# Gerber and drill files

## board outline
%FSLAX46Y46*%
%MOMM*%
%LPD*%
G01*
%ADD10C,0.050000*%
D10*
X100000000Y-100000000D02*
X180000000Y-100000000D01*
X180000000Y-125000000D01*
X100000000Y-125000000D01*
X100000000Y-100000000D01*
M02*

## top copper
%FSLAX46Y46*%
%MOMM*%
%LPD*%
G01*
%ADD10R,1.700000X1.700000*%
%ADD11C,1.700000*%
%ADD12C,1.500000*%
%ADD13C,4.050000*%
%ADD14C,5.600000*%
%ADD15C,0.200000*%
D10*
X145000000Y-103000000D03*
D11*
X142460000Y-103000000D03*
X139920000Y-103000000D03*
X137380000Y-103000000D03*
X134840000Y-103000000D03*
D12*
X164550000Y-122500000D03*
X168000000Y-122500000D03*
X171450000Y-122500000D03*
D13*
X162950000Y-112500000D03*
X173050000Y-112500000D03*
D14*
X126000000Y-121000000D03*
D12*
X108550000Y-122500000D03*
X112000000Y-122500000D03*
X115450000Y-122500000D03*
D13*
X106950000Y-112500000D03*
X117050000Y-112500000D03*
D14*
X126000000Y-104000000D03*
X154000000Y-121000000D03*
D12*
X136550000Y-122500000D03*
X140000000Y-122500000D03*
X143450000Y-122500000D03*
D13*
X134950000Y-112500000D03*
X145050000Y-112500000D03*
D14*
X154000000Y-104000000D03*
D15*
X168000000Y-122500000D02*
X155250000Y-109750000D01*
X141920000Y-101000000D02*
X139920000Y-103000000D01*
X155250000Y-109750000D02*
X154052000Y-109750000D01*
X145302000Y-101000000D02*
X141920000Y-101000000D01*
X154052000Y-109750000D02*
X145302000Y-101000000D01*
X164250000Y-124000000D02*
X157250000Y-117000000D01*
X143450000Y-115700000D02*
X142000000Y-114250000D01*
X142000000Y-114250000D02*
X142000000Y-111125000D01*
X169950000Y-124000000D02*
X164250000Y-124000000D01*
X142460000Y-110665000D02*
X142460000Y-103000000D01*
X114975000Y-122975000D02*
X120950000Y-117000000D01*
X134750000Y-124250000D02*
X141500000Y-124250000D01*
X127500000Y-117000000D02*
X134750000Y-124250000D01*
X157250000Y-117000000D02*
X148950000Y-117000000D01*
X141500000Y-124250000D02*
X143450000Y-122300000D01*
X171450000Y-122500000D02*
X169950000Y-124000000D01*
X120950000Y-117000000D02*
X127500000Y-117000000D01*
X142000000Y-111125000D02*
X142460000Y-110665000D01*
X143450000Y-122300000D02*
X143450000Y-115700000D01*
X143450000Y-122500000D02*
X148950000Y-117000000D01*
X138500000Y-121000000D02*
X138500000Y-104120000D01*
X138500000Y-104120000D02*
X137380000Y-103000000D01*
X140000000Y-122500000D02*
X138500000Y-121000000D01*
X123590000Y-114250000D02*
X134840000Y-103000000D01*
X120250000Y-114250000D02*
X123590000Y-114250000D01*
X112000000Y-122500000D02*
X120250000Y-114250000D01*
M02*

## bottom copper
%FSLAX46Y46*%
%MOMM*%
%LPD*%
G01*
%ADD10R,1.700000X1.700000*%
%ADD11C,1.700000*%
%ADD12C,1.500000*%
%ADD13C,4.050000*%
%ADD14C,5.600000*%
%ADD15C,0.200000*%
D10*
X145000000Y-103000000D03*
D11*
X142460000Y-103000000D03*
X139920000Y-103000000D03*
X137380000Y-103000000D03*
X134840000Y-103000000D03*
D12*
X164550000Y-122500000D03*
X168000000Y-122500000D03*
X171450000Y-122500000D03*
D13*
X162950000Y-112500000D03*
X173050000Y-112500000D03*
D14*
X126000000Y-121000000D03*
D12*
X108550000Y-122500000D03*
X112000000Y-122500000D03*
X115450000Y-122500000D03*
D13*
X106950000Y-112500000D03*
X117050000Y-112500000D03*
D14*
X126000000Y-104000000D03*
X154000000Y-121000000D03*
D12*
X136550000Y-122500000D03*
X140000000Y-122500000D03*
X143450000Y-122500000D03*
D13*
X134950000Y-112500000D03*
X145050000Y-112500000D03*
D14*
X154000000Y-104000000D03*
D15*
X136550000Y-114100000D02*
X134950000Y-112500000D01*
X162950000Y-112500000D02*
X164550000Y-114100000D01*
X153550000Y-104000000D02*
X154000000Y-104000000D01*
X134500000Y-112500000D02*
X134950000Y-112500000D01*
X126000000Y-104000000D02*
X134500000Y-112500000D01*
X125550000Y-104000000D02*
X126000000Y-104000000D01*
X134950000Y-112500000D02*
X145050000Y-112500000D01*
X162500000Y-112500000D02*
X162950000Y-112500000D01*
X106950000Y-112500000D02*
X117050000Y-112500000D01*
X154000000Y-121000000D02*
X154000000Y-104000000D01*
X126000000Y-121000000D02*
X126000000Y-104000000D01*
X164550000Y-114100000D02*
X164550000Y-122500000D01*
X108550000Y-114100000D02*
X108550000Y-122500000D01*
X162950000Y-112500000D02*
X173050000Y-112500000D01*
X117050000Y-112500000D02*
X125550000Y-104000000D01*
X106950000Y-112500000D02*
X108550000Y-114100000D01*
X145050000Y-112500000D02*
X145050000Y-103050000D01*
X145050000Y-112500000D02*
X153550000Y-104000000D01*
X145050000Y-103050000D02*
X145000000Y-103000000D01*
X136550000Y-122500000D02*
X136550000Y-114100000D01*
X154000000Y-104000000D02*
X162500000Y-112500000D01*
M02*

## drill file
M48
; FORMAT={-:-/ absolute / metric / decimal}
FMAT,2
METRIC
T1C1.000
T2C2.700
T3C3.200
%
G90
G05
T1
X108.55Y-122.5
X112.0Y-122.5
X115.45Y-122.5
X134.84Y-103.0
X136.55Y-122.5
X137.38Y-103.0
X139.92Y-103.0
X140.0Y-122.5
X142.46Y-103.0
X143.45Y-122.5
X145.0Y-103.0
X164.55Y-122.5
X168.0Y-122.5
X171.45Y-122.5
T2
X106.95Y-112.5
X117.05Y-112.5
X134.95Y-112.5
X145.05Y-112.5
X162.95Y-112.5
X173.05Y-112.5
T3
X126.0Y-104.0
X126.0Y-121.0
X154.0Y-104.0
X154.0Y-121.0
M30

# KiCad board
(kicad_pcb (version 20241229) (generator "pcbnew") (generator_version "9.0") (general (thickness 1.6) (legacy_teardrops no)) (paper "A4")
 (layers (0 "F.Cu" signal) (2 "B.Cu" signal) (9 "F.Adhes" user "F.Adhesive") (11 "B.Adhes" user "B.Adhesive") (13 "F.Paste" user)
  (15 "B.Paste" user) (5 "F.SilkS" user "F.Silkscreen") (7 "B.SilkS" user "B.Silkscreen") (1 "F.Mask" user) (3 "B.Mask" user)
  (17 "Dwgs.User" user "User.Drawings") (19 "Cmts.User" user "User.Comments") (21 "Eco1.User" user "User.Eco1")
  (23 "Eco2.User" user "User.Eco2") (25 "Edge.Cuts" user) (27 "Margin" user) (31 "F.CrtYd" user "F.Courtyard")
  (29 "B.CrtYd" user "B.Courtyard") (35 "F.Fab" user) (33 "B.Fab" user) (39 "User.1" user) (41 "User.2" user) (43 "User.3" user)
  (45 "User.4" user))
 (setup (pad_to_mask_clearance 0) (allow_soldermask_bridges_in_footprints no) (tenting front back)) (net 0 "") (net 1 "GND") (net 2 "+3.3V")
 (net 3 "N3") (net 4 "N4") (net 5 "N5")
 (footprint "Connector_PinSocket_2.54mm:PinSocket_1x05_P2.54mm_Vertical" (layer "F.Cu") (at 145 103 -90)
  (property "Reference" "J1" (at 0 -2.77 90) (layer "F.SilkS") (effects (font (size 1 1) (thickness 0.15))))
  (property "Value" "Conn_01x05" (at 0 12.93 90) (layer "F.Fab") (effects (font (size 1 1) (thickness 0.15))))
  (pad "1" thru_hole rect (at 0 0 270) (size 1.7 1.7) (drill 1) (layers "*.Cu" "*.Mask") (remove_unused_layers no) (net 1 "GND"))
  (pad "2" thru_hole circle (at 0 2.54 270) (size 1.7 1.7) (drill 1) (layers "*.Cu" "*.Mask") (remove_unused_layers no) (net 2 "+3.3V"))
  (pad "3" thru_hole circle (at 0 5.08 270) (size 1.7 1.7) (drill 1) (layers "*.Cu" "*.Mask") (remove_unused_layers no) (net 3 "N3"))
  (pad "4" thru_hole circle (at 0 7.62 270) (size 1.7 1.7) (drill 1) (layers "*.Cu" "*.Mask") (remove_unused_layers no) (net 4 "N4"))
  (pad "5" thru_hole circle (at 0 10.16 270) (size 1.7 1.7) (drill 1) (layers "*.Cu" "*.Mask") (remove_unused_layers no) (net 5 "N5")))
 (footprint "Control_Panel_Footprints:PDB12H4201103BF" (layer "F.Cu") (at 165.5 122.5)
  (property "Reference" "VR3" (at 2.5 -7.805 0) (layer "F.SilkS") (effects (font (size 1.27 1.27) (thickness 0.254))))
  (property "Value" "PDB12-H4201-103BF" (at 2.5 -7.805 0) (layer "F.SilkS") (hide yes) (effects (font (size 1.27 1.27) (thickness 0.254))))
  (pad "1" thru_hole circle (at -0.95 0) (size 1.5 1.5) (drill 1) (layers "*.Cu" "*.Mask") (remove_unused_layers no) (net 1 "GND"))
  (pad "2" thru_hole circle (at 2.5 0) (size 1.5 1.5) (drill 1) (layers "*.Cu" "*.Mask") (remove_unused_layers no) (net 3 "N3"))
  (pad "3" thru_hole circle (at 5.95 0) (size 1.5 1.5) (drill 1) (layers "*.Cu" "*.Mask") (remove_unused_layers no) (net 2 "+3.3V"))
  (pad "MH1" thru_hole circle (at -2.55 -10) (size 4.05 4.05) (drill 2.7) (layers "*.Cu" "*.Mask") (remove_unused_layers no) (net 1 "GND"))
  (pad "MH2" thru_hole circle (at 7.55 -10) (size 4.05 4.05) (drill 2.7) (layers "*.Cu" "*.Mask") (remove_unused_layers no) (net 1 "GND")))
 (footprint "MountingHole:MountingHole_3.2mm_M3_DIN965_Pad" (layer "F.Cu") (at 126 121)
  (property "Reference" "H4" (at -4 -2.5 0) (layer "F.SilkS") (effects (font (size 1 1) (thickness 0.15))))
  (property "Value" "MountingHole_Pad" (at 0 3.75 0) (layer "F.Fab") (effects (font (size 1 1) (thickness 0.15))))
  (pad "1" thru_hole circle (at 0 0) (size 5.6 5.6) (drill 3.2) (layers "*.Cu" "*.Mask") (remove_unused_layers no) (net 1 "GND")
   (zone_connect 2)))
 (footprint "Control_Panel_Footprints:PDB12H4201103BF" (layer "F.Cu") (at 109.5 122.5)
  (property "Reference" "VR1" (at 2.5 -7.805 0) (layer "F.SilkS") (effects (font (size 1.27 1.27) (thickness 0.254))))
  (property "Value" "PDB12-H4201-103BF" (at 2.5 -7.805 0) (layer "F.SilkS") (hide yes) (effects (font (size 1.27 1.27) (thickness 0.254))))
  (pad "1" thru_hole circle (at -0.95 0) (size 1.5 1.5) (drill 1) (layers "*.Cu" "*.Mask") (remove_unused_layers no) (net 1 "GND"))
  (pad "2" thru_hole circle (at 2.5 0) (size 1.5 1.5) (drill 1) (layers "*.Cu" "*.Mask") (remove_unused_layers no) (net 5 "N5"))
  (pad "3" thru_hole circle (at 5.95 0) (size 1.5 1.5) (drill 1) (layers "*.Cu" "*.Mask") (remove_unused_layers no) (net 2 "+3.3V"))
  (pad "MH1" thru_hole circle (at -2.55 -10) (size 4.05 4.05) (drill 2.7) (layers "*.Cu" "*.Mask") (remove_unused_layers no) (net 1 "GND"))
  (pad "MH2" thru_hole circle (at 7.55 -10) (size 4.05 4.05) (drill 2.7) (layers "*.Cu" "*.Mask") (remove_unused_layers no) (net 1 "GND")))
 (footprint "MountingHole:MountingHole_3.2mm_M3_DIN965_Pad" (layer "F.Cu") (at 126 104)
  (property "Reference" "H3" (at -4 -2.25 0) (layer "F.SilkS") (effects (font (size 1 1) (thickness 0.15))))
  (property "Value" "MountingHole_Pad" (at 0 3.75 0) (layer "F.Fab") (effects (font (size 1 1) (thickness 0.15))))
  (pad "1" thru_hole circle (at 0 0) (size 5.6 5.6) (drill 3.2) (layers "*.Cu" "*.Mask") (remove_unused_layers no) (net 1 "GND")
   (zone_connect 2)))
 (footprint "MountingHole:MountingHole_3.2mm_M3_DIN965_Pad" (layer "F.Cu") (at 154 121)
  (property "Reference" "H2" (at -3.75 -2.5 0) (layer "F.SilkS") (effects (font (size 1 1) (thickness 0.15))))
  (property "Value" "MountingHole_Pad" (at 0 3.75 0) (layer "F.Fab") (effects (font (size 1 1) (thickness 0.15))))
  (pad "1" thru_hole circle (at 0 0) (size 5.6 5.6) (drill 3.2) (layers "*.Cu" "*.Mask") (remove_unused_layers no) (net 1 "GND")
   (zone_connect 2)))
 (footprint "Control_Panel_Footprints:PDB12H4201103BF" (layer "F.Cu") (at 137.5 122.5)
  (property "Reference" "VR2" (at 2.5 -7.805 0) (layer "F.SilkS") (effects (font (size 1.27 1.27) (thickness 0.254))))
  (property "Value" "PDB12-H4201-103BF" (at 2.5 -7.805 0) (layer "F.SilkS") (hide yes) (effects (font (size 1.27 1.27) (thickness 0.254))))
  (pad "1" thru_hole circle (at -0.95 0) (size 1.5 1.5) (drill 1) (layers "*.Cu" "*.Mask") (remove_unused_layers no) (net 1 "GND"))
  (pad "2" thru_hole circle (at 2.5 0) (size 1.5 1.5) (drill 1) (layers "*.Cu" "*.Mask") (remove_unused_layers no) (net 4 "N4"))
  (pad "3" thru_hole circle (at 5.95 0) (size 1.5 1.5) (drill 1) (layers "*.Cu" "*.Mask") (remove_unused_layers no) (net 2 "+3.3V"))
  (pad "MH1" thru_hole circle (at -2.55 -10) (size 4.05 4.05) (drill 2.7) (layers "*.Cu" "*.Mask") (remove_unused_layers no) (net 1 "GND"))
  (pad "MH2" thru_hole circle (at 7.55 -10) (size 4.05 4.05) (drill 2.7) (layers "*.Cu" "*.Mask") (remove_unused_layers no) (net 1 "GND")))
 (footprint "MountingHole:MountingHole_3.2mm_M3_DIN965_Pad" (layer "F.Cu") (at 154 104)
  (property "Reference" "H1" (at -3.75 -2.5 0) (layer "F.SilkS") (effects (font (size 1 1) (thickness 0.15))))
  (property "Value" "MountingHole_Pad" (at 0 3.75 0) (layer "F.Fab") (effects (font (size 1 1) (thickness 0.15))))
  (pad "1" thru_hole circle (at 0 0) (size 5.6 5.6) (drill 3.2) (layers "*.Cu" "*.Mask") (remove_unused_layers no) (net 1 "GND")
   (zone_connect 2)))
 (gr_rect (start 100 100) (end 180 125) (stroke (width 0.05) (type solid)) (fill no) (layer "Edge.Cuts"))
 (segment (start 136.55 114.1) (end 134.95 112.5) (width 0.2) (layer "B.Cu") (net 1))
 (segment (start 162.95 112.5) (end 164.55 114.1) (width 0.2) (layer "B.Cu") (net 1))
 (segment (start 153.55 104) (end 154 104) (width 0.2) (layer "B.Cu") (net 1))
 (segment (start 134.5 112.5) (end 134.95 112.5) (width 0.2) (layer "B.Cu") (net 1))
 (segment (start 126 104) (end 134.5 112.5) (width 0.2) (layer "B.Cu") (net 1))
 (segment (start 125.55 104) (end 126 104) (width 0.2) (layer "B.Cu") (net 1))
 (segment (start 134.95 112.5) (end 145.05 112.5) (width 0.2) (layer "B.Cu") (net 1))
 (segment (start 162.5 112.5) (end 162.95 112.5) (width 0.2) (layer "B.Cu") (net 1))
 (segment (start 106.95 112.5) (end 117.05 112.5) (width 0.2) (layer "B.Cu") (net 1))
 (segment (start 154 121) (end 154 104) (width 0.2) (layer "B.Cu") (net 1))
 (segment (start 126 121) (end 126 104) (width 0.2) (layer "B.Cu") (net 1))
 (segment (start 164.55 114.1) (end 164.55 122.5) (width 0.2) (layer "B.Cu") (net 1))
 (segment (start 108.55 114.1) (end 108.55 122.5) (width 0.2) (layer "B.Cu") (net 1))
 (segment (start 162.95 112.5) (end 173.05 112.5) (width 0.2) (layer "B.Cu") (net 1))
 (segment (start 117.05 112.5) (end 125.55 104) (width 0.2) (layer "B.Cu") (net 1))
 (segment (start 106.95 112.5) (end 108.55 114.1) (width 0.2) (layer "B.Cu") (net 1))
 (segment (start 145.05 112.5) (end 145.05 103.05) (width 0.2) (layer "B.Cu") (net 1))
 (segment (start 145.05 112.5) (end 153.55 104) (width 0.2) (layer "B.Cu") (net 1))
 (segment (start 145.05 103.05) (end 145 103) (width 0.2) (layer "B.Cu") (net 1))
 (segment (start 136.55 122.5) (end 136.55 114.1) (width 0.2) (layer "B.Cu") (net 1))
 (segment (start 154 104) (end 162.5 112.5) (width 0.2) (layer "B.Cu") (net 1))
 (segment (start 168 122.5) (end 155.25 109.75) (width 0.2) (layer "F.Cu") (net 3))
 (segment (start 141.92 101) (end 139.92 103) (width 0.2) (layer "F.Cu") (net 3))
 (segment (start 155.25 109.75) (end 154.052 109.75) (width 0.2) (layer "F.Cu") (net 3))
 (segment (start 145.302 101) (end 141.92 101) (width 0.2) (layer "F.Cu") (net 3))
 (segment (start 154.052 109.75) (end 145.302 101) (width 0.2) (layer "F.Cu") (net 3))
 (segment (start 164.25 124) (end 157.25 117) (width 0.2) (layer "F.Cu") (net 2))
 (segment (start 143.45 115.7) (end 142 114.25) (width 0.2) (layer "F.Cu") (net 2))
 (segment (start 142 114.25) (end 142 111.125) (width 0.2) (layer "F.Cu") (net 2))
 (segment (start 169.95 124) (end 164.25 124) (width 0.2) (layer "F.Cu") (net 2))
 (segment (start 142.46 110.665) (end 142.46 103) (width 0.2) (layer "F.Cu") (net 2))
 (segment (start 114.975 122.975) (end 120.95 117) (width 0.2) (layer "F.Cu") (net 2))
 (segment (start 134.75 124.25) (end 141.5 124.25) (width 0.2) (layer "F.Cu") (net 2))
 (segment (start 127.5 117) (end 134.75 124.25) (width 0.2) (layer "F.Cu") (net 2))
 (segment (start 157.25 117) (end 148.95 117) (width 0.2) (layer "F.Cu") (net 2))
 (segment (start 141.5 124.25) (end 143.45 122.3) (width 0.2) (layer "F.Cu") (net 2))
 (segment (start 171.45 122.5) (end 169.95 124) (width 0.2) (layer "F.Cu") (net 2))
 (segment (start 120.95 117) (end 127.5 117) (width 0.2) (layer "F.Cu") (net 2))
 (segment (start 142 111.125) (end 142.46 110.665) (width 0.2) (layer "F.Cu") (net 2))
 (segment (start 143.45 122.3) (end 143.45 115.7) (width 0.2) (layer "F.Cu") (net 2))
 (segment (start 143.45 122.5) (end 148.95 117) (width 0.2) (layer "F.Cu") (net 2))
 (segment (start 138.5 121) (end 138.5 104.12) (width 0.2) (layer "F.Cu") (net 4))
 (segment (start 138.5 104.12) (end 137.38 103) (width 0.2) (layer "F.Cu") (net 4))
 (segment (start 140 122.5) (end 138.5 121) (width 0.2) (layer "F.Cu") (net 4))
 (segment (start 123.59 114.25) (end 134.84 103) (width 0.2) (layer "F.Cu") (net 5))
 (segment (start 120.25 114.25) (end 123.59 114.25) (width 0.2) (layer "F.Cu") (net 5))
 (segment (start 112 122.5) (end 120.25 114.25) (width 0.2) (layer "F.Cu") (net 5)))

